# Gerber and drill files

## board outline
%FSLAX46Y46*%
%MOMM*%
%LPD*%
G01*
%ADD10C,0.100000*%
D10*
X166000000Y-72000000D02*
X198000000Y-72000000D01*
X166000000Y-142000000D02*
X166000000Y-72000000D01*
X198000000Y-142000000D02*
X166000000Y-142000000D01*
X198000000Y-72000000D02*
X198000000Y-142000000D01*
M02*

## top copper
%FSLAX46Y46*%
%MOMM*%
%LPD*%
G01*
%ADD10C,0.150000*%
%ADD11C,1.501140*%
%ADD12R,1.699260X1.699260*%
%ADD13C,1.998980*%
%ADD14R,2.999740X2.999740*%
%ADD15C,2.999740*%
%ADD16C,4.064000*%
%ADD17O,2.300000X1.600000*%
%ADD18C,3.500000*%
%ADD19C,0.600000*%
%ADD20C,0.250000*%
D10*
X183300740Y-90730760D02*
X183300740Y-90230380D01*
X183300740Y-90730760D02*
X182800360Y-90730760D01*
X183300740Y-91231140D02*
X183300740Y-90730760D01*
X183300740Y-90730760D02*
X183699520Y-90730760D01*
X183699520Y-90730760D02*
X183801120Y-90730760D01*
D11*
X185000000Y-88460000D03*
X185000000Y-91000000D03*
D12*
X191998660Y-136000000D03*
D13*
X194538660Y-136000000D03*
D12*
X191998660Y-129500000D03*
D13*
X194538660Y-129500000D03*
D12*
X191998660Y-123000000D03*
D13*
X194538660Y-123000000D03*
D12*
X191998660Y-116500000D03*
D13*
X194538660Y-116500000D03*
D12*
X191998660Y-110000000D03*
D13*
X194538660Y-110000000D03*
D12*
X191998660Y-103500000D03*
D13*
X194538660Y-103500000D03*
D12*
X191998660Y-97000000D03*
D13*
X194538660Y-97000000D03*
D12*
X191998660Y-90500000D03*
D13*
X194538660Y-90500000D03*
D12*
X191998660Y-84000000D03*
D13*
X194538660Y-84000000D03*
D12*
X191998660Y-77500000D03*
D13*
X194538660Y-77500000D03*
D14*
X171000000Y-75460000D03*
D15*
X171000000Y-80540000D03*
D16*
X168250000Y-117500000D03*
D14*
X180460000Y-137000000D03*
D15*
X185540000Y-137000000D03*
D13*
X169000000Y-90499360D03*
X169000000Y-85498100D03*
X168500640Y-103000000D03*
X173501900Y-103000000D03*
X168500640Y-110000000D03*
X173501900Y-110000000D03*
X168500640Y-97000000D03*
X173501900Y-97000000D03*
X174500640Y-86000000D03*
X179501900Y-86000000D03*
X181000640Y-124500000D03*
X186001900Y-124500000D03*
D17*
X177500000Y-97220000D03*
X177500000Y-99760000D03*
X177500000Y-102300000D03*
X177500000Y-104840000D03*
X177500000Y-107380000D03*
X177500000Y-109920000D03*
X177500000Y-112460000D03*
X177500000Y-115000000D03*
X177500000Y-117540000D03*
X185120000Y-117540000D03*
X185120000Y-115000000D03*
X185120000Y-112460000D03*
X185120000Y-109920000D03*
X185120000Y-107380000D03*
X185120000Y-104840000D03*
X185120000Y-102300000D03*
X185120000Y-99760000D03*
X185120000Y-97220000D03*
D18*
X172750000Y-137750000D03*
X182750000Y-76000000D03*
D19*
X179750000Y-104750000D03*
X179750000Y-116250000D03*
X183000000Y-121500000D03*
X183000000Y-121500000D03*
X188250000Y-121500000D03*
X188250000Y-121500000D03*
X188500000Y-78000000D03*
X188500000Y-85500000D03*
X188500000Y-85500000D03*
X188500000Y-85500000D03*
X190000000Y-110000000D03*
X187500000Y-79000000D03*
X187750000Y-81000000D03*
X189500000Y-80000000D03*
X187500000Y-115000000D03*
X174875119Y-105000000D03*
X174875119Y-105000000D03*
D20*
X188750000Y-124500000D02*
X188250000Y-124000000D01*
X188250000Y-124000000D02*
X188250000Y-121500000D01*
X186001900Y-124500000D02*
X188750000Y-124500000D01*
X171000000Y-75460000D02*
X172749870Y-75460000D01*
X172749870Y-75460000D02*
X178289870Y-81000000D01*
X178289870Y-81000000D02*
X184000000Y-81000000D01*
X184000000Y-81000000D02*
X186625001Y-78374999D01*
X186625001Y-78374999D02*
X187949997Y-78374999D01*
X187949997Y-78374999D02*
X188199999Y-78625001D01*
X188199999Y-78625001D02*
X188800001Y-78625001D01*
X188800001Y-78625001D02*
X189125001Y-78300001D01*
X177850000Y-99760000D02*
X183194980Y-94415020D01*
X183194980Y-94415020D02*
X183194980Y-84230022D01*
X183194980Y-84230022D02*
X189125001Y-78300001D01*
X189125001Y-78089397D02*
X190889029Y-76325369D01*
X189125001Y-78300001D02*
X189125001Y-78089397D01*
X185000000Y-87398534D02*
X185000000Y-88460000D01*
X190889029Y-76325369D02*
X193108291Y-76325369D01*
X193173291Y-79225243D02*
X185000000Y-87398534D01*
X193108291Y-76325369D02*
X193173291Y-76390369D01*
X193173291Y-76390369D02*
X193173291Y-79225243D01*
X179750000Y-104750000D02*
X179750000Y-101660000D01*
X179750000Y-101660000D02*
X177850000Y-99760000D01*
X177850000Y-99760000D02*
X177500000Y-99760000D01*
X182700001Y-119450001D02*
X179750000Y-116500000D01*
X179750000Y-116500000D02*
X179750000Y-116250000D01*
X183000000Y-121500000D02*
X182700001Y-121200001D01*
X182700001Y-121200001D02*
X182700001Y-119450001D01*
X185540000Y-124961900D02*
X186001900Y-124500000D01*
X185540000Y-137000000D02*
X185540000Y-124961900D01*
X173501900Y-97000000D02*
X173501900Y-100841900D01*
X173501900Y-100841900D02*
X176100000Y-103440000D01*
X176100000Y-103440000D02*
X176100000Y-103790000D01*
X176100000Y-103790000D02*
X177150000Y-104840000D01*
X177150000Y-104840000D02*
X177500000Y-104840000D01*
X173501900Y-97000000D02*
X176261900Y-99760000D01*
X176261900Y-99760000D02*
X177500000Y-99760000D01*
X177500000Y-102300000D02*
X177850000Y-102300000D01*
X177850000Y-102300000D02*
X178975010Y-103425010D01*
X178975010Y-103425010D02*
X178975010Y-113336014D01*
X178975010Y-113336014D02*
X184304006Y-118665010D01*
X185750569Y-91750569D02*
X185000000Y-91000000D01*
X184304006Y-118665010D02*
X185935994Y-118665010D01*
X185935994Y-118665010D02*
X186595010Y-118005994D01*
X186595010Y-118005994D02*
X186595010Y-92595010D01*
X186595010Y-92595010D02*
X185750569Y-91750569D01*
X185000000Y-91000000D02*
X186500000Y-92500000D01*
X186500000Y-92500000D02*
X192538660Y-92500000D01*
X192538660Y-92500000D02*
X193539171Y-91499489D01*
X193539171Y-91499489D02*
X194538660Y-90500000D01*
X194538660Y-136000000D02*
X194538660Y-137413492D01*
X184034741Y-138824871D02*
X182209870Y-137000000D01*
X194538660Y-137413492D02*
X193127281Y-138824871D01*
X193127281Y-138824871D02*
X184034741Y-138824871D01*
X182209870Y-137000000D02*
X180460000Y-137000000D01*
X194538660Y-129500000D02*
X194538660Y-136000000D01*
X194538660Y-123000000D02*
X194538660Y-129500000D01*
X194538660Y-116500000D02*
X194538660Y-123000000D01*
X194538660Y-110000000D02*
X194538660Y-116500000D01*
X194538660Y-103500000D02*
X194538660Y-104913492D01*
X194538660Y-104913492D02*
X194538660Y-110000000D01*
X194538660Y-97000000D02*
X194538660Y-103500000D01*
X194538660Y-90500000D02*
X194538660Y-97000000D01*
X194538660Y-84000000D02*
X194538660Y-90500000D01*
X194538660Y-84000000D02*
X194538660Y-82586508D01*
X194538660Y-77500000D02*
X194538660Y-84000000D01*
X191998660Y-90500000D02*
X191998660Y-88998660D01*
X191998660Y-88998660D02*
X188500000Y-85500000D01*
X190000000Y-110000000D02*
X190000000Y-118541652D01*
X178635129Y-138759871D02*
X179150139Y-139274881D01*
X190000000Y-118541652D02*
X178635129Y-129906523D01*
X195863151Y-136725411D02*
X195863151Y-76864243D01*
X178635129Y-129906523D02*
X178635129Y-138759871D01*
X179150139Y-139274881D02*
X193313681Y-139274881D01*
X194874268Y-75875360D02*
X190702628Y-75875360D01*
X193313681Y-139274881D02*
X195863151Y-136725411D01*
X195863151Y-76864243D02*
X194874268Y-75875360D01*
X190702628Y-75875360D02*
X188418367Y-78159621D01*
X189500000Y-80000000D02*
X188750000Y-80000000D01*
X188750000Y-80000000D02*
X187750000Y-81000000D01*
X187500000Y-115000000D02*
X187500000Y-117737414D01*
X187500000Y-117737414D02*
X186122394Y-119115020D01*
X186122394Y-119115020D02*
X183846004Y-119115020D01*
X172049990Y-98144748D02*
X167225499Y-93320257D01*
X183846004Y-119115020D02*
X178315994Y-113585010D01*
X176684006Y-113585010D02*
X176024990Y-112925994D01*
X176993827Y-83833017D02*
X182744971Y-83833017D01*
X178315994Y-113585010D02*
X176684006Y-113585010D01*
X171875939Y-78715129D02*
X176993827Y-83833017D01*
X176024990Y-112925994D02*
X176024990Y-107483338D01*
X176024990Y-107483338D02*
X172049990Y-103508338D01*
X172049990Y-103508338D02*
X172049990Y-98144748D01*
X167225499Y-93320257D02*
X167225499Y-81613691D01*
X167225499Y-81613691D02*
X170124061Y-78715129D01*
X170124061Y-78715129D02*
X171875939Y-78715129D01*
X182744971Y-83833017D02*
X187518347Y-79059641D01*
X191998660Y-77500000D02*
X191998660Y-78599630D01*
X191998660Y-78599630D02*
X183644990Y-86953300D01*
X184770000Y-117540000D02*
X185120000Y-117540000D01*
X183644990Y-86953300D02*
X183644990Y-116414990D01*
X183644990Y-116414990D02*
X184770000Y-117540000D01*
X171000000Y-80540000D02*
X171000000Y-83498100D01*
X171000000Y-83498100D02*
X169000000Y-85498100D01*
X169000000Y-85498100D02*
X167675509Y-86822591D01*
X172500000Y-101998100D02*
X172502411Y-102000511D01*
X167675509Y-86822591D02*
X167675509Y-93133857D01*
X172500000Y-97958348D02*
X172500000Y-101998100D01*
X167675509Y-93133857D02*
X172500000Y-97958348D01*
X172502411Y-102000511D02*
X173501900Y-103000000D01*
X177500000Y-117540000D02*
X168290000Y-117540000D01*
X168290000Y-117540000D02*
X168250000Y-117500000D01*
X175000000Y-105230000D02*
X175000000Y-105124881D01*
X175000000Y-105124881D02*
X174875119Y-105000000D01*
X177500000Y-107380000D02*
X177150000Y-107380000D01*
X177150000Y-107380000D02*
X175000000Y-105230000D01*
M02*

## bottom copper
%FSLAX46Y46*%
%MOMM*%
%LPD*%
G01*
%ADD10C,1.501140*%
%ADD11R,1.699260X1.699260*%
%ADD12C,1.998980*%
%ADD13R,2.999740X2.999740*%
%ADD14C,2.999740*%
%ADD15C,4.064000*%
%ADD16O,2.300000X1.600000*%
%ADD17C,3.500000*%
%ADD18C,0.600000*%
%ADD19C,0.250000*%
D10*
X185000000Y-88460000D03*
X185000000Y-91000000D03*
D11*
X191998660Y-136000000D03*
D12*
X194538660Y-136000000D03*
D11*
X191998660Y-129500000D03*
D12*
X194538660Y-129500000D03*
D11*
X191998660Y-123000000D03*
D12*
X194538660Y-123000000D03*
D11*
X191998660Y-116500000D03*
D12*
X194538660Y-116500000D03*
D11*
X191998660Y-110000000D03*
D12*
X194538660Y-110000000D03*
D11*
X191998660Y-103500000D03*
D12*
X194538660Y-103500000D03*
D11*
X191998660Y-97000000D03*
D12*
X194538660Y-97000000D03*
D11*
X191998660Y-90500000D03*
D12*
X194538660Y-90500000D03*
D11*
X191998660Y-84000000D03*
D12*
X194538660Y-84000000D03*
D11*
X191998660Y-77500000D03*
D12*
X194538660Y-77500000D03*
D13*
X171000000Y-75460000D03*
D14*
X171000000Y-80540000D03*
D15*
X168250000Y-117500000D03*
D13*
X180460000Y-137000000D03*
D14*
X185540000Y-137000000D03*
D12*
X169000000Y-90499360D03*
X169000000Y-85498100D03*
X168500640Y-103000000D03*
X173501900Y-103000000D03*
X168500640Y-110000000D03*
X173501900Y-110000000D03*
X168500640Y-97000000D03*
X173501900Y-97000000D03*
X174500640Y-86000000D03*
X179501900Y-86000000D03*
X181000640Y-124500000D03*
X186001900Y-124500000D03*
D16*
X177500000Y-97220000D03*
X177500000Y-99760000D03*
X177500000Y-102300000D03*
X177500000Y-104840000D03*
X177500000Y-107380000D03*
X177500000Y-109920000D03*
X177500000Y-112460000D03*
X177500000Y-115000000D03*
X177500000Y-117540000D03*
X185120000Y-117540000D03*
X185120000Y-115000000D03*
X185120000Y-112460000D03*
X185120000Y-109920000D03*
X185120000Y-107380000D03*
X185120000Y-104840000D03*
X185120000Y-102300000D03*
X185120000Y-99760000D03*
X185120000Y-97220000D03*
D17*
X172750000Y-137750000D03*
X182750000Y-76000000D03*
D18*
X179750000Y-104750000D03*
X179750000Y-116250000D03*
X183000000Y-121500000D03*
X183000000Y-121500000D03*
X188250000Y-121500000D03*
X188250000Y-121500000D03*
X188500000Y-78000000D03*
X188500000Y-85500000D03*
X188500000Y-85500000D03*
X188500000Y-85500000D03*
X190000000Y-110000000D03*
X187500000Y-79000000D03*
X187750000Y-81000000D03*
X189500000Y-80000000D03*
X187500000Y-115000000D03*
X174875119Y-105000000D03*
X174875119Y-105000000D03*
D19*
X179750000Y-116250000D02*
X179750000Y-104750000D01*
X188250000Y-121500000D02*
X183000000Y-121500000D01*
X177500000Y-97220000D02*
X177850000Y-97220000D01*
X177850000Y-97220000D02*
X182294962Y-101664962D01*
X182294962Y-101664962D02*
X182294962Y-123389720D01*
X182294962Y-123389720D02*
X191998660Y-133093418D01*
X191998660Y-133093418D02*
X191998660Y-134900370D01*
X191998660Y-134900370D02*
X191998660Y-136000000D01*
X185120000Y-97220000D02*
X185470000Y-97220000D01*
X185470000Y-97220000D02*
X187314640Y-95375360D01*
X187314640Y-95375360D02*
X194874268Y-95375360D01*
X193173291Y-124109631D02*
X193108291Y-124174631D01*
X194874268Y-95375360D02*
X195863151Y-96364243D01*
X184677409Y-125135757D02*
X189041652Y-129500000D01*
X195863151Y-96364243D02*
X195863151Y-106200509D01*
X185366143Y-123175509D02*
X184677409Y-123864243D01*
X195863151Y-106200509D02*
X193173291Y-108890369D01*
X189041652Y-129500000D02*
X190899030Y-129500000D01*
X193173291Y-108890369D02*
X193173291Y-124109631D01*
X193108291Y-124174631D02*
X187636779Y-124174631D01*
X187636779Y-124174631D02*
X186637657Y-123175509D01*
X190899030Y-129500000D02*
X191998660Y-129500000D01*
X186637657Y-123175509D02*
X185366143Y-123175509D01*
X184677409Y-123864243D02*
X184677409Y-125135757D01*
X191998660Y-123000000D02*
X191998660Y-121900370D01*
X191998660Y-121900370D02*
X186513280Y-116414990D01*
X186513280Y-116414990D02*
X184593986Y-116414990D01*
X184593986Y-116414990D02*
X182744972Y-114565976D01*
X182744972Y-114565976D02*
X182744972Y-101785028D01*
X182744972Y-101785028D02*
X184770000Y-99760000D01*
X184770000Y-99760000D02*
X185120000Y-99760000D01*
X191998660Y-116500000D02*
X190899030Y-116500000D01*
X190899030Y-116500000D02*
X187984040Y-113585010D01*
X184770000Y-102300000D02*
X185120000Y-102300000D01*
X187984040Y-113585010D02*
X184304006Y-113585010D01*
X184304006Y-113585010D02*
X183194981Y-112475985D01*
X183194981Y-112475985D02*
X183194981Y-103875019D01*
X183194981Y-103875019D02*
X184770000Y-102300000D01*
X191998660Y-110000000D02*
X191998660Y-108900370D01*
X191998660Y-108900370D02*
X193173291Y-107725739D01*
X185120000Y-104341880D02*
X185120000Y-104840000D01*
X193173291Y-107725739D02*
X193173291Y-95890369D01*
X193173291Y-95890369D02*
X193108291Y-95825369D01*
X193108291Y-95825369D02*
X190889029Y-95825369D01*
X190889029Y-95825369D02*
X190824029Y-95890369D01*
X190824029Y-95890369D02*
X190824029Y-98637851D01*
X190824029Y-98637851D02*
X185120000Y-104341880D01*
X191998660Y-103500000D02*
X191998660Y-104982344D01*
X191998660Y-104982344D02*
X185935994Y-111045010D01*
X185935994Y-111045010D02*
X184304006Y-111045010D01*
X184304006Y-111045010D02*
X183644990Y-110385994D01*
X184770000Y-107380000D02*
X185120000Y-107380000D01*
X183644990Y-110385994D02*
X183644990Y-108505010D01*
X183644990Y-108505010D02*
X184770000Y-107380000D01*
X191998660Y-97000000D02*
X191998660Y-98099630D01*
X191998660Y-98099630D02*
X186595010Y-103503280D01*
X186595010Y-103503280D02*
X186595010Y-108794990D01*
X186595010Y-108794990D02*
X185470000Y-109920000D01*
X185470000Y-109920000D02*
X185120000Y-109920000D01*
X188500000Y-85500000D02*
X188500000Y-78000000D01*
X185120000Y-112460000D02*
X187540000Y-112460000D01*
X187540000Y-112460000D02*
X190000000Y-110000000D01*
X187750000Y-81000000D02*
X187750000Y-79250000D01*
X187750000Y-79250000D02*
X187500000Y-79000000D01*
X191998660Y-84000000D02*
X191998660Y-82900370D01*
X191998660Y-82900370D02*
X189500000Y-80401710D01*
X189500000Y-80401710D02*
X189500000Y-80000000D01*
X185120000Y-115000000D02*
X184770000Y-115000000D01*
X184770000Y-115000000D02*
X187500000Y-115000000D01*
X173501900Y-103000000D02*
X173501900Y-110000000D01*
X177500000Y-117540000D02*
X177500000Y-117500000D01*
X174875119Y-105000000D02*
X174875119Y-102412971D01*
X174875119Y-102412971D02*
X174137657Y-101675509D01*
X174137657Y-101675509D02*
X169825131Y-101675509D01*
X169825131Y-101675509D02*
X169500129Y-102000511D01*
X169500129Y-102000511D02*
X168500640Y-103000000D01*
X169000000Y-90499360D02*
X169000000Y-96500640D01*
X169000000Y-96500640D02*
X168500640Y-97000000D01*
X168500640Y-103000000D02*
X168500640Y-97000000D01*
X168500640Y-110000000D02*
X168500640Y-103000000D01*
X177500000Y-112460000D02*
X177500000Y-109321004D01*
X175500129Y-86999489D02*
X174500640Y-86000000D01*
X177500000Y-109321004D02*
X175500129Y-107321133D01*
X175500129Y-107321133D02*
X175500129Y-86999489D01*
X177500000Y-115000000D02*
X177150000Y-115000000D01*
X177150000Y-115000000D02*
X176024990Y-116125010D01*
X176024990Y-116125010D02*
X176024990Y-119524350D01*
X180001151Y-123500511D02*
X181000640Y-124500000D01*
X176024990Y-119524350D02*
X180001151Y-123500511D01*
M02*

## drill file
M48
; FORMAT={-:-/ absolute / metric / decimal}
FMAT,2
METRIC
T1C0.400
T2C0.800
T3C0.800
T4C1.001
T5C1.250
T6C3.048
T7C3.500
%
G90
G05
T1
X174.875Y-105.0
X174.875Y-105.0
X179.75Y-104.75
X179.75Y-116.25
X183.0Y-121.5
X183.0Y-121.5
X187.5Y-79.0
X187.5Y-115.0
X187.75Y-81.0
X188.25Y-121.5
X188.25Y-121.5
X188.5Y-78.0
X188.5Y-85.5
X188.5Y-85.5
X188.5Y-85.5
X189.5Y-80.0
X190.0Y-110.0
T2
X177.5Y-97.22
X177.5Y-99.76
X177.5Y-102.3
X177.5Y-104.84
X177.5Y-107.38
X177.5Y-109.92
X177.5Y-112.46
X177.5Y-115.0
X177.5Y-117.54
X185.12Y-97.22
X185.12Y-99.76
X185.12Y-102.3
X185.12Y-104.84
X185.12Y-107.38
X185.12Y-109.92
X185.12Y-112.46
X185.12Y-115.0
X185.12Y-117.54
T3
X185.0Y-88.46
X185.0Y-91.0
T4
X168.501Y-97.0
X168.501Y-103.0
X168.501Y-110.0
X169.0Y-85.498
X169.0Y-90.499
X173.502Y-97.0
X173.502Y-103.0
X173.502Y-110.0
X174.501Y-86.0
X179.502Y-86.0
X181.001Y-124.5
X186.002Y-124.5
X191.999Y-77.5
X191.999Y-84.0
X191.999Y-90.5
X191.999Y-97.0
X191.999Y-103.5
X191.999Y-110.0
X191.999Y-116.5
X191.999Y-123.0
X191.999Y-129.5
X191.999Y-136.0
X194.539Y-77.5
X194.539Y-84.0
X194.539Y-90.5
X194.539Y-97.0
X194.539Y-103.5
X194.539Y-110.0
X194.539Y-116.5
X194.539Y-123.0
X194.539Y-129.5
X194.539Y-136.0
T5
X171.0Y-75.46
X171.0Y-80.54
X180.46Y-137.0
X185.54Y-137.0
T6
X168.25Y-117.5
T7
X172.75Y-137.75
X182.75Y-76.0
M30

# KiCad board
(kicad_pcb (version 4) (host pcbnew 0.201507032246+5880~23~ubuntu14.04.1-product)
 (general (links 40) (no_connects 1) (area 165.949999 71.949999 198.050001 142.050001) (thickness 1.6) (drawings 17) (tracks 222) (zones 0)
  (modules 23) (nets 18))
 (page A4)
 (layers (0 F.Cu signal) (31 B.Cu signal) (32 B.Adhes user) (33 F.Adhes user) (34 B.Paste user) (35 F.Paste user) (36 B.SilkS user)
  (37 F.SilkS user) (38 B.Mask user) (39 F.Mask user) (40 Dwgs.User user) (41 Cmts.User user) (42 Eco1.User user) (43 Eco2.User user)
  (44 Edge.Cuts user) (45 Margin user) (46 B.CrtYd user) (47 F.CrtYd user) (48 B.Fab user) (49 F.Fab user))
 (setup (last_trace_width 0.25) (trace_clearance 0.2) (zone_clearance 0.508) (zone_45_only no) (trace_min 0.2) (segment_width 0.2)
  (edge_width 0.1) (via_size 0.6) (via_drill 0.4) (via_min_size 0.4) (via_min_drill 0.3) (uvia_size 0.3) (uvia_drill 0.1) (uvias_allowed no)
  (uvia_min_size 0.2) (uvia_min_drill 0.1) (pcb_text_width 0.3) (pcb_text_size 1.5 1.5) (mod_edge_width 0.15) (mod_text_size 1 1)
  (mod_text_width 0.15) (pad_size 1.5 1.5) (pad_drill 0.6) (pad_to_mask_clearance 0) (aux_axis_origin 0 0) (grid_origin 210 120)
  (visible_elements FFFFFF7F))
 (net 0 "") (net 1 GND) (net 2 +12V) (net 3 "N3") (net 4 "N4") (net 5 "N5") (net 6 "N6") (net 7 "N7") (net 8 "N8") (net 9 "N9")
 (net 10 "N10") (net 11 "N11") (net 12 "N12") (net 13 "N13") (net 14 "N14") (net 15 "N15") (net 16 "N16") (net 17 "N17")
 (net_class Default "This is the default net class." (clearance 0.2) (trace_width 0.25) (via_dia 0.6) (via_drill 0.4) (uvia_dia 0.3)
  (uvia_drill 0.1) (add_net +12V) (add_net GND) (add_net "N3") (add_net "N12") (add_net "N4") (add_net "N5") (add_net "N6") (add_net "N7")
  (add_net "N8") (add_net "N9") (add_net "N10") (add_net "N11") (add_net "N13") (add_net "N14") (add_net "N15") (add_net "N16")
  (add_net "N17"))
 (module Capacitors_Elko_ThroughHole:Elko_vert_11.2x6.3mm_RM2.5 (layer F.Cu) (at 185 91 90)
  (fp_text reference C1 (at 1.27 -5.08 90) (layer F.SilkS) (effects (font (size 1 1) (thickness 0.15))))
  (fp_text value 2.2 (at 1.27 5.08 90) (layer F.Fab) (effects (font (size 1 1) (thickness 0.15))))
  (fp_line (start 0.26924 -1.69926) (end 0.76962 -1.69926) (layer F.Cu) (width 0.15))
  (fp_line (start 0.26924 -1.69926) (end 0.26924 -2.19964) (layer F.Cu) (width 0.15))
  (fp_line (start -0.23114 -1.69926) (end 0.26924 -1.69926) (layer F.Cu) (width 0.15))
  (fp_line (start 0.26924 -1.69926) (end 0.26924 -1.30048) (layer F.Cu) (width 0.15))
  (fp_line (start 0.26924 -1.30048) (end 0.26924 -1.19888) (layer F.Cu) (width 0.15))
  (pad 2 thru_hole circle (at 2.54 0 90) (size 1.50114 1.50114) (drill 0.8001) (layers *.Cu *.Mask F.SilkS) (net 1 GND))
  (pad 1 thru_hole circle (at 0 0 90) (size 1.50114 1.50114) (drill 0.8001) (layers *.Cu *.Mask F.SilkS) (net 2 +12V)))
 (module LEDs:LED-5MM (layer F.Cu) (at 192 136)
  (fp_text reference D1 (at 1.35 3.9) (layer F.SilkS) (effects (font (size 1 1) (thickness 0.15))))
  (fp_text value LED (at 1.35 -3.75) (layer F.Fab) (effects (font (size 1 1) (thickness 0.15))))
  (pad 1 thru_hole rect (at -0.00134 0 90) (size 1.69926 1.69926) (drill 1.00076) (layers *.Cu *.Mask F.SilkS) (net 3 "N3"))
  (pad 2 thru_hole circle (at 2.53866 0) (size 1.99898 1.99898) (drill 1.00076) (layers *.Cu *.Mask F.SilkS) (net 2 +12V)))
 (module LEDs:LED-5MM (layer F.Cu) (at 192 129.5)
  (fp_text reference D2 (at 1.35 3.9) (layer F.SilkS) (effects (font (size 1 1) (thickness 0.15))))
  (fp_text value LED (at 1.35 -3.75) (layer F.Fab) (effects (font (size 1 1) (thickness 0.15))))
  (pad 1 thru_hole rect (at -0.00134 0 90) (size 1.69926 1.69926) (drill 1.00076) (layers *.Cu *.Mask F.SilkS) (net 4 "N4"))
  (pad 2 thru_hole circle (at 2.53866 0) (size 1.99898 1.99898) (drill 1.00076) (layers *.Cu *.Mask F.SilkS) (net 2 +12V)))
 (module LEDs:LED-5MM (layer F.Cu) (at 192 123)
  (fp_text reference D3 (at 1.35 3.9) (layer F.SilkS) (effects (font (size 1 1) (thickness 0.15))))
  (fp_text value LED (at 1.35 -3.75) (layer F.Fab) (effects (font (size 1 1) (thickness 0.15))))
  (pad 1 thru_hole rect (at -0.00134 0 90) (size 1.69926 1.69926) (drill 1.00076) (layers *.Cu *.Mask F.SilkS) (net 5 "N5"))
  (pad 2 thru_hole circle (at 2.53866 0) (size 1.99898 1.99898) (drill 1.00076) (layers *.Cu *.Mask F.SilkS) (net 2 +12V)))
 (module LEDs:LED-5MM (layer F.Cu) (at 192 116.5)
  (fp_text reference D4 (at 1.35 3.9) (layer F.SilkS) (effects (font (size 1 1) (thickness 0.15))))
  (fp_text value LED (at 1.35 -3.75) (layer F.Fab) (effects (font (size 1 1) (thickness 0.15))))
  (pad 1 thru_hole rect (at -0.00134 0 90) (size 1.69926 1.69926) (drill 1.00076) (layers *.Cu *.Mask F.SilkS) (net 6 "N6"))
  (pad 2 thru_hole circle (at 2.53866 0) (size 1.99898 1.99898) (drill 1.00076) (layers *.Cu *.Mask F.SilkS) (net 2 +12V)))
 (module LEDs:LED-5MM (layer F.Cu) (at 192 110)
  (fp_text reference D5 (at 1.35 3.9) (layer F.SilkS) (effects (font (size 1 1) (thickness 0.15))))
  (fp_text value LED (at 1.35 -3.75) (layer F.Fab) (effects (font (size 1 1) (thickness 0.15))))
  (pad 1 thru_hole rect (at -0.00134 0 90) (size 1.69926 1.69926) (drill 1.00076) (layers *.Cu *.Mask F.SilkS) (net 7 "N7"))
  (pad 2 thru_hole circle (at 2.53866 0) (size 1.99898 1.99898) (drill 1.00076) (layers *.Cu *.Mask F.SilkS) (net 2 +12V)))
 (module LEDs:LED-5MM (layer F.Cu) (at 192 103.5)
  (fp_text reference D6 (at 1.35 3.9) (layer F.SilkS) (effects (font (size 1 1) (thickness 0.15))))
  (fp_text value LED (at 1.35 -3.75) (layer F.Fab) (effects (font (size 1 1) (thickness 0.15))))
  (pad 1 thru_hole rect (at -0.00134 0 90) (size 1.69926 1.69926) (drill 1.00076) (layers *.Cu *.Mask F.SilkS) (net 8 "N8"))
  (pad 2 thru_hole circle (at 2.53866 0) (size 1.99898 1.99898) (drill 1.00076) (layers *.Cu *.Mask F.SilkS) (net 2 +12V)))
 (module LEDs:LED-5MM (layer F.Cu) (at 192 97)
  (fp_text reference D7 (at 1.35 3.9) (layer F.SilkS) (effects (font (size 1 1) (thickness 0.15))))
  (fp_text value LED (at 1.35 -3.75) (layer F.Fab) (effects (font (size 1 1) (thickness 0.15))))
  (pad 1 thru_hole rect (at -0.00134 0 90) (size 1.69926 1.69926) (drill 1.00076) (layers *.Cu *.Mask F.SilkS) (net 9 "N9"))
  (pad 2 thru_hole circle (at 2.53866 0) (size 1.99898 1.99898) (drill 1.00076) (layers *.Cu *.Mask F.SilkS) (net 2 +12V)))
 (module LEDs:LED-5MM (layer F.Cu) (at 192 90.5)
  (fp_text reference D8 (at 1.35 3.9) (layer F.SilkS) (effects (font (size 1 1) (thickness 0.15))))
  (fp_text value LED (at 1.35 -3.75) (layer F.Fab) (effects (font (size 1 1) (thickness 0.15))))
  (pad 1 thru_hole rect (at -0.00134 0 90) (size 1.69926 1.69926) (drill 1.00076) (layers *.Cu *.Mask F.SilkS) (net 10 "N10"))
  (pad 2 thru_hole circle (at 2.53866 0) (size 1.99898 1.99898) (drill 1.00076) (layers *.Cu *.Mask F.SilkS) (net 2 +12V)))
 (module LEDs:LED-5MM (layer F.Cu) (at 192 84)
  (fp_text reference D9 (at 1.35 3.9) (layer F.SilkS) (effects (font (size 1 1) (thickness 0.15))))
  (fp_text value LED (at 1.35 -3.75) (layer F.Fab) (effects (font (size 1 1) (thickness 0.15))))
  (pad 1 thru_hole rect (at -0.00134 0 90) (size 1.69926 1.69926) (drill 1.00076) (layers *.Cu *.Mask F.SilkS) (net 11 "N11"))
  (pad 2 thru_hole circle (at 2.53866 0) (size 1.99898 1.99898) (drill 1.00076) (layers *.Cu *.Mask F.SilkS) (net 2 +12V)))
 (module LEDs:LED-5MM (layer F.Cu) (at 192 77.5)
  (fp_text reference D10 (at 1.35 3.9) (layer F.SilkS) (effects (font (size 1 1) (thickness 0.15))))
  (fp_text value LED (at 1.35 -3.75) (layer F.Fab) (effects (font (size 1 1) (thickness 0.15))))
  (pad 1 thru_hole rect (at -0.00134 0 90) (size 1.69926 1.69926) (drill 1.00076) (layers *.Cu *.Mask F.SilkS) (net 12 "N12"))
  (pad 2 thru_hole circle (at 2.53866 0) (size 1.99898 1.99898) (drill 1.00076) (layers *.Cu *.Mask F.SilkS) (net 2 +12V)))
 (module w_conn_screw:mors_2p (layer F.Cu) (at 171 78 270)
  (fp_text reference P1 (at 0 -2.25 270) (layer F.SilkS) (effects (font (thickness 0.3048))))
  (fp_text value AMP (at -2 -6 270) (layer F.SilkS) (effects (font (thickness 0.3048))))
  (pad 1 thru_hole rect (at -2.54 0 270) (size 2.99974 2.99974) (drill 1.24968) (layers *.Cu *.Mask F.SilkS) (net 1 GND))
  (pad 2 thru_hole circle (at 2.54 0 270) (size 2.99974 2.99974) (drill 1.24968) (layers *.Cu *.Mask F.SilkS) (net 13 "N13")))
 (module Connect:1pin (layer F.Cu) (at 168.25 117.5)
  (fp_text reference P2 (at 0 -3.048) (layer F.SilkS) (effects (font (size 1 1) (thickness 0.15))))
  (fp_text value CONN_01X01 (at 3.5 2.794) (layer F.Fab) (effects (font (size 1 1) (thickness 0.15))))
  (pad 1 thru_hole circle (at 0 0) (size 4.064 4.064) (drill 3.048) (layers *.Cu *.Mask F.SilkS) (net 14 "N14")))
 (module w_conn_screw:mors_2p (layer F.Cu) (at 183 137)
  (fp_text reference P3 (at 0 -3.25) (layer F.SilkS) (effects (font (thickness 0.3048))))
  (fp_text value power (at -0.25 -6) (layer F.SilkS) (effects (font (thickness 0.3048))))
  (pad 1 thru_hole rect (at -2.54 0) (size 2.99974 2.99974) (drill 1.24968) (layers *.Cu *.Mask F.SilkS) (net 2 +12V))
  (pad 2 thru_hole circle (at 2.54 0) (size 2.99974 2.99974) (drill 1.24968) (layers *.Cu *.Mask F.SilkS) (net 1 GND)))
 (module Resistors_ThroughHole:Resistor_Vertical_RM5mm (layer F.Cu) (at 169 88 90)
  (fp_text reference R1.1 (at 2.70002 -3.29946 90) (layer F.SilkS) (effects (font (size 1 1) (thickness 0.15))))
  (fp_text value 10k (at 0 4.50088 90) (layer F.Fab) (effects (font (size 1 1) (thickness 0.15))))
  (pad 1 thru_hole circle (at -2.49936 0 90) (size 1.99898 1.99898) (drill 1.00076) (layers *.Cu *.SilkS *.Mask) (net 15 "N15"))
  (pad 2 thru_hole circle (at 2.5019 0 90) (size 1.99898 1.99898) (drill 1.00076) (layers *.Cu *.SilkS *.Mask) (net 13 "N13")))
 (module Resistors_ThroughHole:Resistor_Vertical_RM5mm (layer F.Cu) (at 171 103)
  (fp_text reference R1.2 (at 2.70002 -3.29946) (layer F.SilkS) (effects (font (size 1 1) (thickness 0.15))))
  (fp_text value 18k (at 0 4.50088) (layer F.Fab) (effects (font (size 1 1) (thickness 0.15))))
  (pad 1 thru_hole circle (at -2.49936 0) (size 1.99898 1.99898) (drill 1.00076) (layers *.Cu *.SilkS *.Mask) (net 15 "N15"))
  (pad 2 thru_hole circle (at 2.5019 0) (size 1.99898 1.99898) (drill 1.00076) (layers *.Cu *.SilkS *.Mask) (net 13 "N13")))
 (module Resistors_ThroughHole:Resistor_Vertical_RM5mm (layer F.Cu) (at 171 110)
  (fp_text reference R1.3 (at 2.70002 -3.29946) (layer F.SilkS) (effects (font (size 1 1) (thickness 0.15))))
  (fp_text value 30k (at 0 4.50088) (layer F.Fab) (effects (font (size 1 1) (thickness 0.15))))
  (pad 1 thru_hole circle (at -2.49936 0) (size 1.99898 1.99898) (drill 1.00076) (layers *.Cu *.SilkS *.Mask) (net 15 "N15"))
  (pad 2 thru_hole circle (at 2.5019 0) (size 1.99898 1.99898) (drill 1.00076) (layers *.Cu *.SilkS *.Mask) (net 13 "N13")))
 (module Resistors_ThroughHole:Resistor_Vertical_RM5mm (layer F.Cu) (at 171 97)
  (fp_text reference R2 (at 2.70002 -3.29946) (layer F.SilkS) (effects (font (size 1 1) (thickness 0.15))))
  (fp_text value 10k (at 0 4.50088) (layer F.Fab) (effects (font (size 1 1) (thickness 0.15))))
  (pad 1 thru_hole circle (at -2.49936 0) (size 1.99898 1.99898) (drill 1.00076) (layers *.Cu *.SilkS *.Mask) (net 15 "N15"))
  (pad 2 thru_hole circle (at 2.5019 0) (size 1.99898 1.99898) (drill 1.00076) (layers *.Cu *.SilkS *.Mask) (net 1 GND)))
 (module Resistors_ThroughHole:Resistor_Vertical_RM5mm (layer F.Cu) (at 177 86)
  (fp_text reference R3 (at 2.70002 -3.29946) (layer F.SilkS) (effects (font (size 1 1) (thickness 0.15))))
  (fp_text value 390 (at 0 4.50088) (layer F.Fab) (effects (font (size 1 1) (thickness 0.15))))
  (pad 1 thru_hole circle (at -2.49936 0) (size 1.99898 1.99898) (drill 1.00076) (layers *.Cu *.SilkS *.Mask) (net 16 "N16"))
  (pad 2 thru_hole circle (at 2.5019 0) (size 1.99898 1.99898) (drill 1.00076) (layers *.Cu *.SilkS *.Mask) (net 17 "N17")))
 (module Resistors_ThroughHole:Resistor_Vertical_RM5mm (layer F.Cu) (at 183.5 124.5)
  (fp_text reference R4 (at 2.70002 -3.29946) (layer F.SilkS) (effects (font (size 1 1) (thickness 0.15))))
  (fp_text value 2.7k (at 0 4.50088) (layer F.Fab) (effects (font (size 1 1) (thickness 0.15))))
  (pad 1 thru_hole circle (at -2.49936 0) (size 1.99898 1.99898) (drill 1.00076) (layers *.Cu *.SilkS *.Mask) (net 17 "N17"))
  (pad 2 thru_hole circle (at 2.5019 0) (size 1.99898 1.99898) (drill 1.00076) (layers *.Cu *.SilkS *.Mask) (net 1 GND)))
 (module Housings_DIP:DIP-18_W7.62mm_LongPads (layer F.Cu) (at 177.5 97.22)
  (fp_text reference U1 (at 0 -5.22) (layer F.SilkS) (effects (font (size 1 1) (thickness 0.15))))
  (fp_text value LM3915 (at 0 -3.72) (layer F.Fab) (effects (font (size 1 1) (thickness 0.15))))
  (pad 1 thru_hole oval (at 0 0) (size 2.3 1.6) (drill 0.8) (layers *.Cu *.Mask F.SilkS) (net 3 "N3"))
  (pad 2 thru_hole oval (at 0 2.54) (size 2.3 1.6) (drill 0.8) (layers *.Cu *.Mask F.SilkS) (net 1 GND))
  (pad 3 thru_hole oval (at 0 5.08) (size 2.3 1.6) (drill 0.8) (layers *.Cu *.Mask F.SilkS) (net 2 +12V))
  (pad 4 thru_hole oval (at 0 7.62) (size 2.3 1.6) (drill 0.8) (layers *.Cu *.Mask F.SilkS) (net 1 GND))
  (pad 5 thru_hole oval (at 0 10.16) (size 2.3 1.6) (drill 0.8) (layers *.Cu *.Mask F.SilkS) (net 15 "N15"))
  (pad 6 thru_hole oval (at 0 12.7) (size 2.3 1.6) (drill 0.8) (layers *.Cu *.Mask F.SilkS) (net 16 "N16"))
  (pad 7 thru_hole oval (at 0 15.24) (size 2.3 1.6) (drill 0.8) (layers *.Cu *.Mask F.SilkS) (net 16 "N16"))
  (pad 8 thru_hole oval (at 0 17.78) (size 2.3 1.6) (drill 0.8) (layers *.Cu *.Mask F.SilkS) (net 17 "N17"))
  (pad 9 thru_hole oval (at 0 20.32) (size 2.3 1.6) (drill 0.8) (layers *.Cu *.Mask F.SilkS) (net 14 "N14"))
  (pad 10 thru_hole oval (at 7.62 20.32) (size 2.3 1.6) (drill 0.8) (layers *.Cu *.Mask F.SilkS) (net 12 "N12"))
  (pad 11 thru_hole oval (at 7.62 17.78) (size 2.3 1.6) (drill 0.8) (layers *.Cu *.Mask F.SilkS) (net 11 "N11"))
  (pad 12 thru_hole oval (at 7.62 15.24) (size 2.3 1.6) (drill 0.8) (layers *.Cu *.Mask F.SilkS) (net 10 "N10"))
  (pad 13 thru_hole oval (at 7.62 12.7) (size 2.3 1.6) (drill 0.8) (layers *.Cu *.Mask F.SilkS) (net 9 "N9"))
  (pad 14 thru_hole oval (at 7.62 10.16) (size 2.3 1.6) (drill 0.8) (layers *.Cu *.Mask F.SilkS) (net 8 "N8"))
  (pad 15 thru_hole oval (at 7.62 7.62) (size 2.3 1.6) (drill 0.8) (layers *.Cu *.Mask F.SilkS) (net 7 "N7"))
  (pad 16 thru_hole oval (at 7.62 5.08) (size 2.3 1.6) (drill 0.8) (layers *.Cu *.Mask F.SilkS) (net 6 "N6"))
  (pad 17 thru_hole oval (at 7.62 2.54) (size 2.3 1.6) (drill 0.8) (layers *.Cu *.Mask F.SilkS) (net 5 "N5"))
  (pad 18 thru_hole oval (at 7.62 0) (size 2.3 1.6) (drill 0.8) (layers *.Cu *.Mask F.SilkS) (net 4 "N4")))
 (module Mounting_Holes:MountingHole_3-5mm (layer F.Cu) (at 172.75 137.75)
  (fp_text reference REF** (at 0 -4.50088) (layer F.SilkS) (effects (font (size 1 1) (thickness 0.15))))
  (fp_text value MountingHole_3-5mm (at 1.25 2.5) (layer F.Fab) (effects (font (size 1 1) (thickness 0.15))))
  (pad 1 thru_hole circle (at 0 0) (size 3.5 3.5) (drill 3.5) (layers)))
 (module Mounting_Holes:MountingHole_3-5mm (layer F.Cu) (at 182.75 76)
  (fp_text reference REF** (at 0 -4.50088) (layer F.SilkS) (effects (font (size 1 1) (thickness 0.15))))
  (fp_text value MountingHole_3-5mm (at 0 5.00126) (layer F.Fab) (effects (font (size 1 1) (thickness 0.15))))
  (pad 1 thru_hole circle (at 0 0) (size 3.5 3.5) (drill 3.5) (layers)))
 (gr_line (start 166 72) (end 198 72) (angle 90) (layer Edge.Cuts) (width 0.1))
 (gr_line (start 166 142) (end 166 72) (angle 90) (layer Edge.Cuts) (width 0.1))
 (gr_line (start 198 142) (end 166 142) (angle 90) (layer Edge.Cuts) (width 0.1))
 (gr_line (start 198 72) (end 198 142) (angle 90) (layer Edge.Cuts) (width 0.1))
 (segment (start 170 125) (end 170 126.75) (width 0.25) (layer F.SilkS) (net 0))
 (segment (start 188.75 124.5) (end 188.25 124) (width 0.25) (layer F.Cu) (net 1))
 (segment (start 188.25 124) (end 188.25 121.5) (width 0.25) (layer F.Cu) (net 1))
 (segment (start 186.0019 124.5) (end 188.75 124.5) (width 0.25) (layer F.Cu) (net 1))
 (segment (start 171 75.46) (end 172.74987 75.46) (width 0.25) (layer F.Cu) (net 1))
 (segment (start 172.74987 75.46) (end 178.28987 81) (width 0.25) (layer F.Cu) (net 1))
 (segment (start 178.28987 81) (end 184 81) (width 0.25) (layer F.Cu) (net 1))
 (segment (start 184 81) (end 186.625001 78.374999) (width 0.25) (layer F.Cu) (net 1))
 (segment (start 186.625001 78.374999) (end 187.949997 78.374999) (width 0.25) (layer F.Cu) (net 1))
 (segment (start 187.949997 78.374999) (end 188.199999 78.625001) (width 0.25) (layer F.Cu) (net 1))
 (segment (start 188.199999 78.625001) (end 188.800001 78.625001) (width 0.25) (layer F.Cu) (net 1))
 (segment (start 188.800001 78.625001) (end 189.125001 78.300001) (width 0.25) (layer F.Cu) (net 1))
 (segment (start 177.85 99.76) (end 183.19498 94.41502) (width 0.25) (layer F.Cu) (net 1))
 (segment (start 183.19498 94.41502) (end 183.19498 84.230022) (width 0.25) (layer F.Cu) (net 1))
 (segment (start 183.19498 84.230022) (end 189.125001 78.300001) (width 0.25) (layer F.Cu) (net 1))
 (segment (start 189.125001 78.089397) (end 190.889029 76.325369) (width 0.25) (layer F.Cu) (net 1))
 (segment (start 189.125001 78.300001) (end 189.125001 78.089397) (width 0.25) (layer F.Cu) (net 1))
 (segment (start 185 87.398534) (end 185 88.46) (width 0.25) (layer F.Cu) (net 1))
 (segment (start 190.889029 76.325369) (end 193.108291 76.325369) (width 0.25) (layer F.Cu) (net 1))
 (segment (start 193.173291 79.225243) (end 185 87.398534) (width 0.25) (layer F.Cu) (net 1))
 (segment (start 193.108291 76.325369) (end 193.173291 76.390369) (width 0.25) (layer F.Cu) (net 1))
 (segment (start 193.173291 76.390369) (end 193.173291 79.225243) (width 0.25) (layer F.Cu) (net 1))
 (segment (start 179.75 104.75) (end 179.75 101.66) (width 0.25) (layer F.Cu) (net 1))
 (segment (start 179.75 101.66) (end 177.85 99.76) (width 0.25) (layer F.Cu) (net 1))
 (segment (start 177.85 99.76) (end 177.5 99.76) (width 0.25) (layer F.Cu) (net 1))
 (segment (start 179.75 116.25) (end 179.75 104.75) (width 0.25) (layer B.Cu) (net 1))
 (via (at 179.75 104.75) (size 0.6) (drill 0.4) (layers F.Cu B.Cu) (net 1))
 (segment (start 182.700001 119.450001) (end 179.75 116.5) (width 0.25) (layer F.Cu) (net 1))
 (segment (start 179.75 116.5) (end 179.75 116.25) (width 0.25) (layer F.Cu) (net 1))
 (via (at 179.75 116.25) (size 0.6) (drill 0.4) (layers F.Cu B.Cu) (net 1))
 (segment (start 183 121.5) (end 182.700001 121.200001) (width 0.25) (layer F.Cu) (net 1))
 (segment (start 182.700001 121.200001) (end 182.700001 119.450001) (width 0.25) (layer F.Cu) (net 1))
 (via (at 183 121.5) (size 0.6) (drill 0.4) (layers F.Cu B.Cu) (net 1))
 (via (at 183 121.5) (size 0.6) (drill 0.4) (layers F.Cu B.Cu) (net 1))
 (segment (start 188.25 121.5) (end 183 121.5) (width 0.25) (layer B.Cu) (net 1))
 (via (at 188.25 121.5) (size 0.6) (drill 0.4) (layers F.Cu B.Cu) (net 1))
 (via (at 188.25 121.5) (size 0.6) (drill 0.4) (layers F.Cu B.Cu) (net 1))
 (segment (start 185.54 124.9619) (end 186.0019 124.5) (width 0.25) (layer F.Cu) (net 1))
 (segment (start 185.54 137) (end 185.54 124.9619) (width 0.25) (layer F.Cu) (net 1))
 (segment (start 173.5019 97) (end 173.5019 100.8419) (width 0.25) (layer F.Cu) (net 1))
 (segment (start 173.5019 100.8419) (end 176.1 103.44) (width 0.25) (layer F.Cu) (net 1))
 (segment (start 176.1 103.44) (end 176.1 103.79) (width 0.25) (layer F.Cu) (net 1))
 (segment (start 176.1 103.79) (end 177.15 104.84) (width 0.25) (layer F.Cu) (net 1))
 (segment (start 177.15 104.84) (end 177.5 104.84) (width 0.25) (layer F.Cu) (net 1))
 (segment (start 173.5019 97) (end 176.2619 99.76) (width 0.25) (layer F.Cu) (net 1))
 (segment (start 176.2619 99.76) (end 177.5 99.76) (width 0.25) (layer F.Cu) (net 1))
 (segment (start 177.5 102.3) (end 177.85 102.3) (width 0.25) (layer F.Cu) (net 2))
 (segment (start 177.85 102.3) (end 178.97501 103.42501) (width 0.25) (layer F.Cu) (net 2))
 (segment (start 178.97501 103.42501) (end 178.97501 113.336014) (width 0.25) (layer F.Cu) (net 2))
 (segment (start 178.97501 113.336014) (end 184.304006 118.66501) (width 0.25) (layer F.Cu) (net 2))
 (segment (start 185.750569 91.750569) (end 185 91) (width 0.25) (layer F.Cu) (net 2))
 (segment (start 184.304006 118.66501) (end 185.935994 118.66501) (width 0.25) (layer F.Cu) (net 2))
 (segment (start 185.935994 118.66501) (end 186.59501 118.005994) (width 0.25) (layer F.Cu) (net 2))
 (segment (start 186.59501 118.005994) (end 186.59501 92.59501) (width 0.25) (layer F.Cu) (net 2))
 (segment (start 186.59501 92.59501) (end 185.750569 91.750569) (width 0.25) (layer F.Cu) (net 2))
 (segment (start 185 91) (end 186.5 92.5) (width 0.25) (layer F.Cu) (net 2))
 (segment (start 186.5 92.5) (end 192.53866 92.5) (width 0.25) (layer F.Cu) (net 2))
 (segment (start 192.53866 92.5) (end 193.539171 91.499489) (width 0.25) (layer F.Cu) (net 2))
 (segment (start 193.539171 91.499489) (end 194.53866 90.5) (width 0.25) (layer F.Cu) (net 2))
 (segment (start 194.53866 136) (end 194.53866 137.413492) (width 0.25) (layer F.Cu) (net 2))
 (segment (start 184.034741 138.824871) (end 182.20987 137) (width 0.25) (layer F.Cu) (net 2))
 (segment (start 194.53866 137.413492) (end 193.127281 138.824871) (width 0.25) (layer F.Cu) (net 2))
 (segment (start 193.127281 138.824871) (end 184.034741 138.824871) (width 0.25) (layer F.Cu) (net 2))
 (segment (start 182.20987 137) (end 180.46 137) (width 0.25) (layer F.Cu) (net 2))
 (segment (start 194.53866 129.5) (end 194.53866 136) (width 0.25) (layer F.Cu) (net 2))
 (segment (start 194.53866 123) (end 194.53866 129.5) (width 0.25) (layer F.Cu) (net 2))
 (segment (start 194.53866 116.5) (end 194.53866 123) (width 0.25) (layer F.Cu) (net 2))
 (segment (start 194.53866 110) (end 194.53866 116.5) (width 0.25) (layer F.Cu) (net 2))
 (segment (start 194.53866 103.5) (end 194.53866 104.913492) (width 0.25) (layer F.Cu) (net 2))
 (segment (start 194.53866 104.913492) (end 194.53866 110) (width 0.25) (layer F.Cu) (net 2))
 (segment (start 194.53866 97) (end 194.53866 103.5) (width 0.25) (layer F.Cu) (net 2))
 (segment (start 194.53866 90.5) (end 194.53866 97) (width 0.25) (layer F.Cu) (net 2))
 (segment (start 194.53866 84) (end 194.53866 90.5) (width 0.25) (layer F.Cu) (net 2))
 (segment (start 194.53866 84) (end 194.53866 82.586508) (width 0.25) (layer F.Cu) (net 2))
 (segment (start 194.53866 77.5) (end 194.53866 84) (width 0.25) (layer F.Cu) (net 2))
 (segment (start 177.5 97.22) (end 177.85 97.22) (width 0.25) (layer B.Cu) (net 3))
 (segment (start 177.85 97.22) (end 182.294962 101.664962) (width 0.25) (layer B.Cu) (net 3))
 (segment (start 182.294962 101.664962) (end 182.294962 123.38972) (width 0.25) (layer B.Cu) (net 3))
 (segment (start 182.294962 123.38972) (end 191.99866 133.093418) (width 0.25) (layer B.Cu) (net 3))
 (segment (start 191.99866 133.093418) (end 191.99866 134.90037) (width 0.25) (layer B.Cu) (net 3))
 (segment (start 191.99866 134.90037) (end 191.99866 136) (width 0.25) (layer B.Cu) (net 3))
 (segment (start 185.12 97.22) (end 185.47 97.22) (width 0.25) (layer B.Cu) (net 4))
 (segment (start 185.47 97.22) (end 187.31464 95.37536) (width 0.25) (layer B.Cu) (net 4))
 (segment (start 187.31464 95.37536) (end 194.874268 95.37536) (width 0.25) (layer B.Cu) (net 4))
 (segment (start 193.173291 124.109631) (end 193.108291 124.174631) (width 0.25) (layer B.Cu) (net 4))
 (segment (start 194.874268 95.37536) (end 195.863151 96.364243) (width 0.25) (layer B.Cu) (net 4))
 (segment (start 184.677409 125.135757) (end 189.041652 129.5) (width 0.25) (layer B.Cu) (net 4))
 (segment (start 195.863151 96.364243) (end 195.863151 106.200509) (width 0.25) (layer B.Cu) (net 4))
 (segment (start 185.366143 123.175509) (end 184.677409 123.864243) (width 0.25) (layer B.Cu) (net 4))
 (segment (start 195.863151 106.200509) (end 193.173291 108.890369) (width 0.25) (layer B.Cu) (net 4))
 (segment (start 189.041652 129.5) (end 190.89903 129.5) (width 0.25) (layer B.Cu) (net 4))
 (segment (start 193.173291 108.890369) (end 193.173291 124.109631) (width 0.25) (layer B.Cu) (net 4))
 (segment (start 193.108291 124.174631) (end 187.636779 124.174631) (width 0.25) (layer B.Cu) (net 4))
 (segment (start 187.636779 124.174631) (end 186.637657 123.175509) (width 0.25) (layer B.Cu) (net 4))
 (segment (start 190.89903 129.5) (end 191.99866 129.5) (width 0.25) (layer B.Cu) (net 4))
 (segment (start 186.637657 123.175509) (end 185.366143 123.175509) (width 0.25) (layer B.Cu) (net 4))
 (segment (start 184.677409 123.864243) (end 184.677409 125.135757) (width 0.25) (layer B.Cu) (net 4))
 (segment (start 191.99866 123) (end 191.99866 121.90037) (width 0.25) (layer B.Cu) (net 5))
 (segment (start 191.99866 121.90037) (end 186.51328 116.41499) (width 0.25) (layer B.Cu) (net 5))
 (segment (start 186.51328 116.41499) (end 184.593986 116.41499) (width 0.25) (layer B.Cu) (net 5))
 (segment (start 184.593986 116.41499) (end 182.744972 114.565976) (width 0.25) (layer B.Cu) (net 5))
 (segment (start 182.744972 114.565976) (end 182.744972 101.785028) (width 0.25) (layer B.Cu) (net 5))
 (segment (start 182.744972 101.785028) (end 184.77 99.76) (width 0.25) (layer B.Cu) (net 5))
 (segment (start 184.77 99.76) (end 185.12 99.76) (width 0.25) (layer B.Cu) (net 5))
 (segment (start 191.99866 116.5) (end 190.89903 116.5) (width 0.25) (layer B.Cu) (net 6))
 (segment (start 190.89903 116.5) (end 187.98404 113.58501) (width 0.25) (layer B.Cu) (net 6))
 (segment (start 184.77 102.3) (end 185.12 102.3) (width 0.25) (layer B.Cu) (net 6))
 (segment (start 187.98404 113.58501) (end 184.304006 113.58501) (width 0.25) (layer B.Cu) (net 6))
 (segment (start 184.304006 113.58501) (end 183.194981 112.475985) (width 0.25) (layer B.Cu) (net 6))
 (segment (start 183.194981 112.475985) (end 183.194981 103.875019) (width 0.25) (layer B.Cu) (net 6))
 (segment (start 183.194981 103.875019) (end 184.77 102.3) (width 0.25) (layer B.Cu) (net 6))
 (segment (start 191.99866 110) (end 191.99866 108.90037) (width 0.25) (layer B.Cu) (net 7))
 (segment (start 191.99866 108.90037) (end 193.173291 107.725739) (width 0.25) (layer B.Cu) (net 7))
 (segment (start 185.12 104.34188) (end 185.12 104.84) (width 0.25) (layer B.Cu) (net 7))
 (segment (start 193.173291 107.725739) (end 193.173291 95.890369) (width 0.25) (layer B.Cu) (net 7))
 (segment (start 193.173291 95.890369) (end 193.108291 95.825369) (width 0.25) (layer B.Cu) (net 7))
 (segment (start 193.108291 95.825369) (end 190.889029 95.825369) (width 0.25) (layer B.Cu) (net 7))
 (segment (start 190.889029 95.825369) (end 190.824029 95.890369) (width 0.25) (layer B.Cu) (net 7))
 (segment (start 190.824029 95.890369) (end 190.824029 98.637851) (width 0.25) (layer B.Cu) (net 7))
 (segment (start 190.824029 98.637851) (end 185.12 104.34188) (width 0.25) (layer B.Cu) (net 7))
 (segment (start 191.99866 103.5) (end 191.99866 104.982344) (width 0.25) (layer B.Cu) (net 8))
 (segment (start 191.99866 104.982344) (end 185.935994 111.04501) (width 0.25) (layer B.Cu) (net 8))
 (segment (start 185.935994 111.04501) (end 184.304006 111.04501) (width 0.25) (layer B.Cu) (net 8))
 (segment (start 184.304006 111.04501) (end 183.64499 110.385994) (width 0.25) (layer B.Cu) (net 8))
 (segment (start 184.77 107.38) (end 185.12 107.38) (width 0.25) (layer B.Cu) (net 8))
 (segment (start 183.64499 110.385994) (end 183.64499 108.50501) (width 0.25) (layer B.Cu) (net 8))
 (segment (start 183.64499 108.50501) (end 184.77 107.38) (width 0.25) (layer B.Cu) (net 8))
 (segment (start 191.99866 97) (end 191.99866 98.09963) (width 0.25) (layer B.Cu) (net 9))
 (segment (start 191.99866 98.09963) (end 186.59501 103.50328) (width 0.25) (layer B.Cu) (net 9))
 (segment (start 186.59501 103.50328) (end 186.59501 108.79499) (width 0.25) (layer B.Cu) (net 9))
 (segment (start 186.59501 108.79499) (end 185.47 109.92) (width 0.25) (layer B.Cu) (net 9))
 (segment (start 185.47 109.92) (end 185.12 109.92) (width 0.25) (layer B.Cu) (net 9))
 (via (at 188.5 78) (size 0.6) (drill 0.4) (layers F.Cu B.Cu) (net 10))
 (via (at 188.5 85.5) (size 0.6) (drill 0.4) (layers F.Cu B.Cu) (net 10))
 (segment (start 188.5 85.5) (end 188.5 78) (width 0.25) (layer B.Cu) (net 10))
 (via (at 188.5 85.5) (size 0.6) (drill 0.4) (layers F.Cu B.Cu) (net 10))
 (segment (start 191.99866 90.5) (end 191.99866 88.99866) (width 0.25) (layer F.Cu) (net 10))
 (segment (start 191.99866 88.99866) (end 188.5 85.5) (width 0.25) (layer F.Cu) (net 10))
 (via (at 188.5 85.5) (size 0.6) (drill 0.4) (layers F.Cu B.Cu) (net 10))
 (segment (start 190 110) (end 190 118.541652) (width 0.25) (layer F.Cu) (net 10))
 (segment (start 178.635129 138.759871) (end 179.150139 139.274881) (width 0.25) (layer F.Cu) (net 10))
 (segment (start 190 118.541652) (end 178.635129 129.906523) (width 0.25) (layer F.Cu) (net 10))
 (segment (start 195.863151 136.725411) (end 195.863151 76.864243) (width 0.25) (layer F.Cu) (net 10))
 (segment (start 178.635129 129.906523) (end 178.635129 138.759871) (width 0.25) (layer F.Cu) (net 10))
 (segment (start 179.150139 139.274881) (end 193.313681 139.274881) (width 0.25) (layer F.Cu) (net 10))
 (segment (start 194.874268 75.87536) (end 190.702628 75.87536) (width 0.25) (layer F.Cu) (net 10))
 (segment (start 193.313681 139.274881) (end 195.863151 136.725411) (width 0.25) (layer F.Cu) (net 10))
 (segment (start 195.863151 76.864243) (end 194.874268 75.87536) (width 0.25) (layer F.Cu) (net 10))
 (segment (start 190.702628 75.87536) (end 188.418367 78.159621) (width 0.25) (layer F.Cu) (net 10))
 (segment (start 185.12 112.46) (end 187.54 112.46) (width 0.25) (layer B.Cu) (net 10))
 (segment (start 187.54 112.46) (end 190 110) (width 0.25) (layer B.Cu) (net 10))
 (via (at 190 110) (size 0.6) (drill 0.4) (layers F.Cu B.Cu) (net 10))
 (segment (start 187.75 81) (end 187.75 79.25) (width 0.25) (layer B.Cu) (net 11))
 (via (at 187.5 79) (size 0.6) (drill 0.4) (layers F.Cu B.Cu) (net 11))
 (segment (start 187.75 79.25) (end 187.5 79) (width 0.25) (layer B.Cu) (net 11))
 (segment (start 189.5 80) (end 188.75 80) (width 0.25) (layer F.Cu) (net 11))
 (segment (start 188.75 80) (end 187.75 81) (width 0.25) (layer F.Cu) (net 11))
 (via (at 187.75 81) (size 0.6) (drill 0.4) (layers F.Cu B.Cu) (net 11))
 (segment (start 191.99866 84) (end 191.99866 82.90037) (width 0.25) (layer B.Cu) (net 11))
 (segment (start 191.99866 82.90037) (end 189.5 80.40171) (width 0.25) (layer B.Cu) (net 11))
 (segment (start 189.5 80.40171) (end 189.5 80) (width 0.25) (layer B.Cu) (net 11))
 (via (at 189.5 80) (size 0.6) (drill 0.4) (layers F.Cu B.Cu) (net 11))
 (segment (start 187.5 115) (end 187.5 117.737414) (width 0.25) (layer F.Cu) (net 11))
 (segment (start 187.5 117.737414) (end 186.122394 119.11502) (width 0.25) (layer F.Cu) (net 11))
 (segment (start 186.122394 119.11502) (end 183.846004 119.11502) (width 0.25) (layer F.Cu) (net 11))
 (segment (start 172.04999 98.144748) (end 167.225499 93.320257) (width 0.25) (layer F.Cu) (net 11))
 (segment (start 183.846004 119.11502) (end 178.315994 113.58501) (width 0.25) (layer F.Cu) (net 11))
 (segment (start 176.684006 113.58501) (end 176.02499 112.925994) (width 0.25) (layer F.Cu) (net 11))
 (segment (start 176.993827 83.833017) (end 182.744971 83.833017) (width 0.25) (layer F.Cu) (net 11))
 (segment (start 178.315994 113.58501) (end 176.684006 113.58501) (width 0.25) (layer F.Cu) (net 11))
 (segment (start 171.875939 78.715129) (end 176.993827 83.833017) (width 0.25) (layer F.Cu) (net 11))
 (segment (start 176.02499 112.925994) (end 176.02499 107.483338) (width 0.25) (layer F.Cu) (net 11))
 (segment (start 176.02499 107.483338) (end 172.04999 103.508338) (width 0.25) (layer F.Cu) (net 11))
 (segment (start 172.04999 103.508338) (end 172.04999 98.144748) (width 0.25) (layer F.Cu) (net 11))
 (segment (start 167.225499 93.320257) (end 167.225499 81.613691) (width 0.25) (layer F.Cu) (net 11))
 (segment (start 167.225499 81.613691) (end 170.124061 78.715129) (width 0.25) (layer F.Cu) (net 11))
 (segment (start 170.124061 78.715129) (end 171.875939 78.715129) (width 0.25) (layer F.Cu) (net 11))
 (segment (start 182.744971 83.833017) (end 187.518347 79.059641) (width 0.25) (layer F.Cu) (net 11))
 (segment (start 185.12 115) (end 184.77 115) (width 0.25) (layer B.Cu) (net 11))
 (segment (start 184.77 115) (end 187.5 115) (width 0.25) (layer B.Cu) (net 11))
 (via (at 187.5 115) (size 0.6) (drill 0.4) (layers F.Cu B.Cu) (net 11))
 (segment (start 191.99866 77.5) (end 191.99866 78.59963) (width 0.25) (layer F.Cu) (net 12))
 (segment (start 191.99866 78.59963) (end 183.64499 86.9533) (width 0.25) (layer F.Cu) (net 12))
 (segment (start 184.77 117.54) (end 185.12 117.54) (width 0.25) (layer F.Cu) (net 12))
 (segment (start 183.64499 86.9533) (end 183.64499 116.41499) (width 0.25) (layer F.Cu) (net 12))
 (segment (start 183.64499 116.41499) (end 184.77 117.54) (width 0.25) (layer F.Cu) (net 12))
 (segment (start 171 80.54) (end 171 83.4981) (width 0.25) (layer F.Cu) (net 13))
 (segment (start 171 83.4981) (end 169 85.4981) (width 0.25) (layer F.Cu) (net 13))
 (segment (start 169 85.4981) (end 167.675509 86.822591) (width 0.25) (layer F.Cu) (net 13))
 (segment (start 172.5 101.9981) (end 172.502411 102.000511) (width 0.25) (layer F.Cu) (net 13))
 (segment (start 167.675509 86.822591) (end 167.675509 93.133857) (width 0.25) (layer F.Cu) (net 13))
 (segment (start 172.5 97.958348) (end 172.5 101.9981) (width 0.25) (layer F.Cu) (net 13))
 (segment (start 167.675509 93.133857) (end 172.5 97.958348) (width 0.25) (layer F.Cu) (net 13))
 (segment (start 172.502411 102.000511) (end 173.5019 103) (width 0.25) (layer F.Cu) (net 13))
 (segment (start 173.5019 103) (end 173.5019 110) (width 0.25) (layer B.Cu) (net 13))
 (segment (start 177.5 117.54) (end 168.29 117.54) (width 0.25) (layer F.Cu) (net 14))
 (segment (start 168.29 117.54) (end 168.25 117.5) (width 0.25) (layer F.Cu) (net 14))
 (segment (start 177.5 117.54) (end 177.5 117.5) (width 0.25) (layer B.Cu) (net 14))
 (segment (start 174.875119 105) (end 174.875119 102.412971) (width 0.25) (layer B.Cu) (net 15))
 (segment (start 174.875119 102.412971) (end 174.137657 101.675509) (width 0.25) (layer B.Cu) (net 15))
 (segment (start 174.137657 101.675509) (end 169.825131 101.675509) (width 0.25) (layer B.Cu) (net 15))
 (segment (start 169.825131 101.675509) (end 169.500129 102.000511) (width 0.25) (layer B.Cu) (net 15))
 (segment (start 169.500129 102.000511) (end 168.50064 103) (width 0.25) (layer B.Cu) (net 15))
 (via (at 174.875119 105) (size 0.6) (drill 0.4) (layers F.Cu B.Cu) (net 15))
 (segment (start 175 105.23) (end 175 105.124881) (width 0.25) (layer F.Cu) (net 15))
 (segment (start 175 105.124881) (end 174.875119 105) (width 0.25) (layer F.Cu) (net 15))
 (via (at 174.875119 105) (size 0.6) (drill 0.4) (layers F.Cu B.Cu) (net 15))
 (segment (start 177.5 107.38) (end 177.15 107.38) (width 0.25) (layer F.Cu) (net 15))
 (segment (start 177.15 107.38) (end 175 105.23) (width 0.25) (layer F.Cu) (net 15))
 (segment (start 169 90.49936) (end 169 96.50064) (width 0.25) (layer B.Cu) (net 15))
 (segment (start 169 96.50064) (end 168.50064 97) (width 0.25) (layer B.Cu) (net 15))
 (segment (start 168.50064 103) (end 168.50064 97) (width 0.25) (layer B.Cu) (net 15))
 (segment (start 168.50064 110) (end 168.50064 103) (width 0.25) (layer B.Cu) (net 15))
 (segment (start 177.5 112.46) (end 177.5 109.321004) (width 0.25) (layer B.Cu) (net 16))
 (segment (start 175.500129 86.999489) (end 174.50064 86) (width 0.25) (layer B.Cu) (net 16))
 (segment (start 177.5 109.321004) (end 175.500129 107.321133) (width 0.25) (layer B.Cu) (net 16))
 (segment (start 175.500129 107.321133) (end 175.500129 86.999489) (width 0.25) (layer B.Cu) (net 16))
 (segment (start 177.5 115) (end 177.15 115) (width 0.25) (layer B.Cu) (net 17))
 (segment (start 177.15 115) (end 176.02499 116.12501) (width 0.25) (layer B.Cu) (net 17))
 (segment (start 176.02499 116.12501) (end 176.02499 119.52435) (width 0.25) (layer B.Cu) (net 17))
 (segment (start 180.001151 123.500511) (end 181.00064 124.5) (width 0.25) (layer B.Cu) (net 17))
 (segment (start 176.02499 119.52435) (end 180.001151 123.500511) (width 0.25) (layer B.Cu) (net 17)))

